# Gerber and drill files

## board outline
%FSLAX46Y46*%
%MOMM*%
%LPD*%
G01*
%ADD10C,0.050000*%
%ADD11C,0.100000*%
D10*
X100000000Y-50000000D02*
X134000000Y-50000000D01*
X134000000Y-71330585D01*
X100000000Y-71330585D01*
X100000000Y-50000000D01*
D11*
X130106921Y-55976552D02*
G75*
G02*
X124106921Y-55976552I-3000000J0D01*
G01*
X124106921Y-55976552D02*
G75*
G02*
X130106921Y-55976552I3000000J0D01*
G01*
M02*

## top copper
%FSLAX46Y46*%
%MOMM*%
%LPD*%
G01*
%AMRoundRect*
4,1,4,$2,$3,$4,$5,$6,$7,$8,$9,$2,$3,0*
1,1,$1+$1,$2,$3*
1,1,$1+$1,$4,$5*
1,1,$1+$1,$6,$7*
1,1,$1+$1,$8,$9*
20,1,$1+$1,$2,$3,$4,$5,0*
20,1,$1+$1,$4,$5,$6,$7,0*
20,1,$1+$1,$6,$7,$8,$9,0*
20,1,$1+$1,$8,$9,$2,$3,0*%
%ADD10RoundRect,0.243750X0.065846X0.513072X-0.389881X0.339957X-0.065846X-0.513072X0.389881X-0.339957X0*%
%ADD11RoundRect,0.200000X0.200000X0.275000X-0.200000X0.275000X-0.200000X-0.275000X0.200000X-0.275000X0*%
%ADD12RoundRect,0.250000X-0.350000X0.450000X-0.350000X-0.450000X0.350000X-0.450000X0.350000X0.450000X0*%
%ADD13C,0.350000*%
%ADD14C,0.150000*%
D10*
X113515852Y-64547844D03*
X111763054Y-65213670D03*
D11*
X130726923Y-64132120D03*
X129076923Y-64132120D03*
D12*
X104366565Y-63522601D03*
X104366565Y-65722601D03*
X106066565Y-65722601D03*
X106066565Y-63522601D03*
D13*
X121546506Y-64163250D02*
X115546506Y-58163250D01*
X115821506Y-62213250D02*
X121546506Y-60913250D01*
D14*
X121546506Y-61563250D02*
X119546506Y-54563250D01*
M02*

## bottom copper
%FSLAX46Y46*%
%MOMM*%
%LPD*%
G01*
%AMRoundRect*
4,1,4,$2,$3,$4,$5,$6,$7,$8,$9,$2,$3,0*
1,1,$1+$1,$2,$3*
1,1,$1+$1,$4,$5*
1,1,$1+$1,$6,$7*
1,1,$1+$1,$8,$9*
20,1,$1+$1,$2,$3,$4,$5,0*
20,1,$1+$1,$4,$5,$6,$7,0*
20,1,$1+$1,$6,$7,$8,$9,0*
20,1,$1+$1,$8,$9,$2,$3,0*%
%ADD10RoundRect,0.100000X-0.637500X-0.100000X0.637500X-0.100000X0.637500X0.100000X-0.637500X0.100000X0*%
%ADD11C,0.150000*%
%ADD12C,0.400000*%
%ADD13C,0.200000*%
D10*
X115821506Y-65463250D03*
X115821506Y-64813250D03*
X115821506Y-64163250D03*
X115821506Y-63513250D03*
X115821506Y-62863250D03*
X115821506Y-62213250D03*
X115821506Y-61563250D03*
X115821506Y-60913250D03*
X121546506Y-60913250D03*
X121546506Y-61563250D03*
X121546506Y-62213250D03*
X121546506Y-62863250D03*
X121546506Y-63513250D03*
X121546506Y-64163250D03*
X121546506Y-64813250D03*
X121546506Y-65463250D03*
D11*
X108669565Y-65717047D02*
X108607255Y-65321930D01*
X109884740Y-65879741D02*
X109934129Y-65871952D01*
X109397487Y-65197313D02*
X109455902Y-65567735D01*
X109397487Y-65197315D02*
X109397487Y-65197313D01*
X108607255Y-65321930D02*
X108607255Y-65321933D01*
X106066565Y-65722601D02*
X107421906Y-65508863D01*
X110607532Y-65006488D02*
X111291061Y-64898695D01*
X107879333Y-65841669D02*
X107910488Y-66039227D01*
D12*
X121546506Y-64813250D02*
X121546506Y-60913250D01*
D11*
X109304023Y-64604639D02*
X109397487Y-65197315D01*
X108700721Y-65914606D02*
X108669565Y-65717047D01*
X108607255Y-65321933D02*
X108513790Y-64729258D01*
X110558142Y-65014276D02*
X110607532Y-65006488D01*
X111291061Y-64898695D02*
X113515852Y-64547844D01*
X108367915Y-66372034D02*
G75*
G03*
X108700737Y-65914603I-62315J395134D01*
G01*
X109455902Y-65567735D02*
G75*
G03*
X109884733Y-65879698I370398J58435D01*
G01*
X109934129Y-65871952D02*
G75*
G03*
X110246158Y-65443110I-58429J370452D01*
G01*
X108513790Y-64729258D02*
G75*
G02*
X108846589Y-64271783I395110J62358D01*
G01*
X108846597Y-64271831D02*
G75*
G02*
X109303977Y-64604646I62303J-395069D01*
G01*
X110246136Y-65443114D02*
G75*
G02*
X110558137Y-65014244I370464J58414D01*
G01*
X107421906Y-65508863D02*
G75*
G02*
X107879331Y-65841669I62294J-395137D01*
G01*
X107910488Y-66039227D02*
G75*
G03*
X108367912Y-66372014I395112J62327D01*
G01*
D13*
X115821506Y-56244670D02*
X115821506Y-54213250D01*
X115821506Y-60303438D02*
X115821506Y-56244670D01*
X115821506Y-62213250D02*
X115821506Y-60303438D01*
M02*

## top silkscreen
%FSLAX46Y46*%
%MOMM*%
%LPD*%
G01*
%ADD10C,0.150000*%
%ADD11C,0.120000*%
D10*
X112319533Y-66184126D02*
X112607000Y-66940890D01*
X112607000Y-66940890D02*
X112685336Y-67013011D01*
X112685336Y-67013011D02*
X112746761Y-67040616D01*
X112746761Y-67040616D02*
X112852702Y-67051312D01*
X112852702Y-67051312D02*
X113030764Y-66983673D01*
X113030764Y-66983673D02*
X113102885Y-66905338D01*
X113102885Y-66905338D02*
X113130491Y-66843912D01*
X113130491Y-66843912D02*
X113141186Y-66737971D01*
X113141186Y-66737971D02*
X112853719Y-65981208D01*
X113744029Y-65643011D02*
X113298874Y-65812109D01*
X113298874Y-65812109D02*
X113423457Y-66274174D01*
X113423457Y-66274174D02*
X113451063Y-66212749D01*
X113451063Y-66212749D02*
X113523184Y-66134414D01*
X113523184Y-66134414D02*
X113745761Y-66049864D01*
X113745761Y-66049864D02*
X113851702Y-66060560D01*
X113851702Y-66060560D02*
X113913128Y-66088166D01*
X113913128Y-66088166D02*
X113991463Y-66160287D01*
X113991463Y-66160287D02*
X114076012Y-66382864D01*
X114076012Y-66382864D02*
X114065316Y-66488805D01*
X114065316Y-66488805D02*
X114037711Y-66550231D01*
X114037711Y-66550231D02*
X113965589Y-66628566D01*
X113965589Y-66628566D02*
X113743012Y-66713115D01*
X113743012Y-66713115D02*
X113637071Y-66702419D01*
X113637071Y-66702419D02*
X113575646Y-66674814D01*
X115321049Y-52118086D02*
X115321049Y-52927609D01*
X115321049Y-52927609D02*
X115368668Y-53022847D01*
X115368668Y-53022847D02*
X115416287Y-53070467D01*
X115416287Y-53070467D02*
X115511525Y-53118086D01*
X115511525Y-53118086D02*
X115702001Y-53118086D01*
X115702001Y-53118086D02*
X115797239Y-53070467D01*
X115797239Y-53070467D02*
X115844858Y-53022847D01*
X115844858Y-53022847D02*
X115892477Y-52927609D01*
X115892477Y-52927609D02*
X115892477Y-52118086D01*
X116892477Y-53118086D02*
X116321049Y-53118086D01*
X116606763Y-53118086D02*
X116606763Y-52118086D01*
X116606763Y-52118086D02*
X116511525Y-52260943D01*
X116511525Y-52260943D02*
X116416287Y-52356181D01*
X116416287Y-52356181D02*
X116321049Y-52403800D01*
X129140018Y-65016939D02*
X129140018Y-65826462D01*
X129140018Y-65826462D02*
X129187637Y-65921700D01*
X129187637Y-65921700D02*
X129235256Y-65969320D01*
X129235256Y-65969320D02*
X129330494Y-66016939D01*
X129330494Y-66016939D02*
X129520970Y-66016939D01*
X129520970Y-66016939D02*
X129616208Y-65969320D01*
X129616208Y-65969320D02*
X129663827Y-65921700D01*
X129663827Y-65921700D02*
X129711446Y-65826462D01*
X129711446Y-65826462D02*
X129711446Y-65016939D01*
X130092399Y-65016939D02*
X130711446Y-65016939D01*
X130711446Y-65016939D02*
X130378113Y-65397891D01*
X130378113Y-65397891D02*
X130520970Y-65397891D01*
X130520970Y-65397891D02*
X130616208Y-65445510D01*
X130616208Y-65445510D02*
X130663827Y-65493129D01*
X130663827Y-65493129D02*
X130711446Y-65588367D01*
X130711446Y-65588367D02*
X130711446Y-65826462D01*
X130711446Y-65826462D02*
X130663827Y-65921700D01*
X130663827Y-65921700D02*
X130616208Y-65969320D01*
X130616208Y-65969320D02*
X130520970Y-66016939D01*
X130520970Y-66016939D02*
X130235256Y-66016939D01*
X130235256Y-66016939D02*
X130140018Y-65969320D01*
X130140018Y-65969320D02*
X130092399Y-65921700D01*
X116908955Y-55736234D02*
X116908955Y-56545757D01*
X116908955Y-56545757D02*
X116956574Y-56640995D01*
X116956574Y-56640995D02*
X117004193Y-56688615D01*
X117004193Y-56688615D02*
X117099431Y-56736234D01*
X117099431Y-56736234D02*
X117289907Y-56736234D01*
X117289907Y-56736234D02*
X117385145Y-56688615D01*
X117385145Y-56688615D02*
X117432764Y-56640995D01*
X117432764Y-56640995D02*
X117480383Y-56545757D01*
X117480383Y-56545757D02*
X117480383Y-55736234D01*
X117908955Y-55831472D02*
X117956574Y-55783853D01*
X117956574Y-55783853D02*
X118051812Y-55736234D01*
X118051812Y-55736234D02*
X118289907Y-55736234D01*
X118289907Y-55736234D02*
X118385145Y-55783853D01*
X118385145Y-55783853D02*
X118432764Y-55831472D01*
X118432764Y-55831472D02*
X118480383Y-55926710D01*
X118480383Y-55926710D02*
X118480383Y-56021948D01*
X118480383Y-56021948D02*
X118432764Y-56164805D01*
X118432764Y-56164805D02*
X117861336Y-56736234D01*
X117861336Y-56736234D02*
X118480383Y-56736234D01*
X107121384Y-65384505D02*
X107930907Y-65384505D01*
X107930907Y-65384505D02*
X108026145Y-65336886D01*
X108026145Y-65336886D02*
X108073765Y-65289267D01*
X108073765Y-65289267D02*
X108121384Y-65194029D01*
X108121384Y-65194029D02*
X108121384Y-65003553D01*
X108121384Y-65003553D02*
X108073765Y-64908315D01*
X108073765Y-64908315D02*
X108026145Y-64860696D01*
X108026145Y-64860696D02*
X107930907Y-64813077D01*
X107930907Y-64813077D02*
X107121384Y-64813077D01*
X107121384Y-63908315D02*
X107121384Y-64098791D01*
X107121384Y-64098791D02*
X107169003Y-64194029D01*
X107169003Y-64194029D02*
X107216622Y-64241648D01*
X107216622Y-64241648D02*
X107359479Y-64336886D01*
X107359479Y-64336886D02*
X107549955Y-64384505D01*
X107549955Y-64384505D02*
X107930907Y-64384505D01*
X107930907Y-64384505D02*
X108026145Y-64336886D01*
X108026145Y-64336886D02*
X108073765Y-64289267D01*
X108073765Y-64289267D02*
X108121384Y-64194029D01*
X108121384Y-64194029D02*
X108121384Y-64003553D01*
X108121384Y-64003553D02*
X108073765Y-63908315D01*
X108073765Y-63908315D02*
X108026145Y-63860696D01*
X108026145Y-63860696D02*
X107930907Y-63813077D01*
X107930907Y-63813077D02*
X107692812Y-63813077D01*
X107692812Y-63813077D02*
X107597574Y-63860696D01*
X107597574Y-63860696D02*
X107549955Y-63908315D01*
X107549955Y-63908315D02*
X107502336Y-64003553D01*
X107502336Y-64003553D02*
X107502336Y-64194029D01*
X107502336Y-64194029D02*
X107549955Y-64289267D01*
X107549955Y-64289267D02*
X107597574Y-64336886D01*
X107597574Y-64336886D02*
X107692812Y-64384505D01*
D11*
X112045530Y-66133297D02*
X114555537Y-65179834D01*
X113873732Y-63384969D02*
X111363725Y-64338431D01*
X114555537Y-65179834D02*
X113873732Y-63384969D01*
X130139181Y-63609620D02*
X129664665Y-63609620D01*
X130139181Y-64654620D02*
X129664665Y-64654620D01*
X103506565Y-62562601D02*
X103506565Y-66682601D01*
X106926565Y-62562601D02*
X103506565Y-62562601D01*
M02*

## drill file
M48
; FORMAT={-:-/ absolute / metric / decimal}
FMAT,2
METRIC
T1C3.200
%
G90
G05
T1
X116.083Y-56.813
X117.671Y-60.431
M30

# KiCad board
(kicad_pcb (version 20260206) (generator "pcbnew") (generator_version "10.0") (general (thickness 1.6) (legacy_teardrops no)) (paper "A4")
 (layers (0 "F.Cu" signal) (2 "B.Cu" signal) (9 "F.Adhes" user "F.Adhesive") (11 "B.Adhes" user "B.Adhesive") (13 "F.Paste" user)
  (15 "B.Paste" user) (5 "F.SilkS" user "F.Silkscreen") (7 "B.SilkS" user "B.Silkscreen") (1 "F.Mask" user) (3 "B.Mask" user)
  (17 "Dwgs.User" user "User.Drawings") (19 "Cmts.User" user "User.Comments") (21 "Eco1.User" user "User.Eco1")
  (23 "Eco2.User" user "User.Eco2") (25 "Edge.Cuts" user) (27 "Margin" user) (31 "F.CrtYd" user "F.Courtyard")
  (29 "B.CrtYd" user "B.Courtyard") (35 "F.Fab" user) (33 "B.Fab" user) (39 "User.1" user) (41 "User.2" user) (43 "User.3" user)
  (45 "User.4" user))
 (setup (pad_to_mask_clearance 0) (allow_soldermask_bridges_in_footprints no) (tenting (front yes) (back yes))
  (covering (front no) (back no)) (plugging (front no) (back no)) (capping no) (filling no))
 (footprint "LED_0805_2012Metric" (layer "F.Cu") (at 112.639453 64.880757 -159.2)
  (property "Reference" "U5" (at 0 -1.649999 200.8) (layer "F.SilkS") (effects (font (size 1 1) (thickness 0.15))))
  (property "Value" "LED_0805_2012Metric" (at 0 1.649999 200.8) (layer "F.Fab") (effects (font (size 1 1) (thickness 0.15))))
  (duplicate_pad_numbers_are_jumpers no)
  (fp_line (start 1 -0.96) (end -1.685 -0.96) (stroke (width 0.12) (type solid)) (layer "F.SilkS"))
  (fp_line (start -1.685 0.96) (end 1 0.96) (stroke (width 0.12) (type solid)) (layer "F.SilkS"))
  (fp_line (start -1.685 -0.96) (end -1.685 0.96) (stroke (width 0.12) (type solid)) (layer "F.SilkS"))
  (pad "1" smd roundrect (at -0.9375 0 200.8) (size 0.975 1.4) (layers "F.Cu" "F.Mask" "F.Paste") (roundrect_rratio 0.25) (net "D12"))
  (pad "2" smd roundrect (at 0.9375 0 200.8) (size 0.975 1.4) (layers "F.Cu" "F.Mask" "F.Paste") (roundrect_rratio 0.25) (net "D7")))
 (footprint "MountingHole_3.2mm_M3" (layer "F.Cu") (at 116.082954 56.813267)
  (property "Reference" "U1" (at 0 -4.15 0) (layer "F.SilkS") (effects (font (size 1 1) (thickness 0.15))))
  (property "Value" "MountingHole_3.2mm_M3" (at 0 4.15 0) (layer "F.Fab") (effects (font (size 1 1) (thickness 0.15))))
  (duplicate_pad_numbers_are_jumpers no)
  (pad "" np_thru_hole circle (at 0 0) (size 3.2 3.2) (drill 3.2) (layers "*.Cu" "*.Mask")))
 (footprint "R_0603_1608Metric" (layer "F.Cu") (at 129.901923 64.13212 180)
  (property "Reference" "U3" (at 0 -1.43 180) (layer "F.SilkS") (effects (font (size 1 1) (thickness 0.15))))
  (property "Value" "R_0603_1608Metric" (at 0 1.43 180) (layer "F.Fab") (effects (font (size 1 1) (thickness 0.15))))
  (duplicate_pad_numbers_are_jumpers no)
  (fp_line (start -0.237258 0.5225) (end 0.237258 0.5225) (stroke (width 0.12) (type solid)) (layer "F.SilkS"))
  (fp_line (start -0.237258 -0.5225) (end 0.237258 -0.5225) (stroke (width 0.12) (type solid)) (layer "F.SilkS"))
  (pad "1" smd roundrect (at -0.825 0 180) (size 0.8 0.95) (layers "F.Cu" "F.Mask" "F.Paste") (roundrect_rratio 0.25) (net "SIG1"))
  (pad "2" smd roundrect (at 0.825 0 180) (size 0.8 0.95) (layers "F.Cu" "F.Mask" "F.Paste") (roundrect_rratio 0.25)))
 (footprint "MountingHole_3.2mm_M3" (layer "F.Cu") (at 117.67086 60.431415)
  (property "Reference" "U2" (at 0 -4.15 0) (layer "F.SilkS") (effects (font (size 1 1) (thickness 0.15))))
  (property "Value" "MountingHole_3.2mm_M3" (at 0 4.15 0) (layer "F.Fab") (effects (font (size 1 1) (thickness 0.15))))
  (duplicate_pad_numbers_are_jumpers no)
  (pad "" np_thru_hole circle (at 0 0) (size 3.2 3.2) (drill 3.2) (layers "*.Cu" "*.Mask")))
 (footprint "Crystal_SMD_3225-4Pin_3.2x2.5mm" (layer "F.Cu") (at 105.216565 64.622601 -90)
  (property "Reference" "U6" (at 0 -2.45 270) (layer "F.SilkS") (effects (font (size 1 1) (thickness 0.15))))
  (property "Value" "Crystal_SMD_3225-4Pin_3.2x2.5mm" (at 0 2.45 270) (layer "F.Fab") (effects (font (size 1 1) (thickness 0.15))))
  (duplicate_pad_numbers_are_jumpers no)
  (fp_line (start -2.06 1.71) (end 2.06 1.71) (stroke (width 0.12) (type solid)) (layer "F.SilkS"))
  (fp_line (start -2.06 -1.71) (end -2.06 1.71) (stroke (width 0.12) (type solid)) (layer "F.SilkS"))
  (pad "1" smd roundrect (at -1.1 0.85 270) (size 1.4 1.2) (layers "F.Cu" "F.Mask" "F.Paste") (roundrect_rratio 0.208333) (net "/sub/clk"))
  (pad "2" smd roundrect (at 1.1 0.85 270) (size 1.4 1.2) (layers "F.Cu" "F.Mask" "F.Paste") (roundrect_rratio 0.208333) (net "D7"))
  (pad "3" smd roundrect (at 1.1 -0.85 270) (size 1.4 1.2) (layers "F.Cu" "F.Mask" "F.Paste") (roundrect_rratio 0.208333) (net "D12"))
  (pad "4" smd roundrect (at -1.1 -0.85 270) (size 1.4 1.2) (layers "F.Cu" "F.Mask" "F.Paste") (roundrect_rratio 0.208333) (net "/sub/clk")))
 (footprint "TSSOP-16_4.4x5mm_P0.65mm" (layer "B.Cu") (at 118.684006 63.18825)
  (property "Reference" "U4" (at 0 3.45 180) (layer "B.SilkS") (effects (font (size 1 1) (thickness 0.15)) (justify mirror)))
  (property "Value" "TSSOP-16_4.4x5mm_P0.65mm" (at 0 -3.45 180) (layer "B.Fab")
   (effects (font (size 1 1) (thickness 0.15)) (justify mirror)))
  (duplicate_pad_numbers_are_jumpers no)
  (pad "1" smd roundrect (at -2.8625 2.275) (size 1.475 0.4) (layers "B.Cu" "B.Mask" "B.Paste") (roundrect_rratio 0.25) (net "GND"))
  (pad "2" smd roundrect (at -2.8625 1.625) (size 1.475 0.4) (layers "B.Cu" "B.Mask" "B.Paste") (roundrect_rratio 0.25) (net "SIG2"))
  (pad "3" smd roundrect (at -2.8625 0.975) (size 1.475 0.4) (layers "B.Cu" "B.Mask" "B.Paste") (roundrect_rratio 0.25) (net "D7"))
  (pad "4" smd roundrect (at -2.8625 0.325) (size 1.475 0.4) (layers "B.Cu" "B.Mask" "B.Paste") (roundrect_rratio 0.25) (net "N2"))
  (pad "5" smd roundrect (at -2.8625 -0.325) (size 1.475 0.4) (layers "B.Cu" "B.Mask" "B.Paste") (roundrect_rratio 0.25) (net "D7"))
  (pad "6" smd roundrect (at -2.8625 -0.975) (size 1.475 0.4) (layers "B.Cu" "B.Mask" "B.Paste") (roundrect_rratio 0.25) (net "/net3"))
  (pad "7" smd roundrect (at -2.8625 -1.625) (size 1.475 0.4) (layers "B.Cu" "B.Mask" "B.Paste") (roundrect_rratio 0.25))
  (pad "8" smd roundrect (at -2.8625 -2.275) (size 1.475 0.4) (layers "B.Cu" "B.Mask" "B.Paste") (roundrect_rratio 0.25) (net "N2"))
  (pad "9" smd roundrect (at 2.8625 -2.275) (size 1.475 0.4) (layers "B.Cu" "B.Mask" "B.Paste") (roundrect_rratio 0.25))
  (pad "10" smd roundrect (at 2.8625 -1.625) (size 1.475 0.4) (layers "B.Cu" "B.Mask" "B.Paste") (roundrect_rratio 0.25) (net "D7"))
  (pad "11" smd roundrect (at 2.8625 -0.975) (size 1.475 0.4) (layers "B.Cu" "B.Mask" "B.Paste") (roundrect_rratio 0.25) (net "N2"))
  (pad "12" smd roundrect (at 2.8625 -0.325) (size 1.475 0.4) (layers "B.Cu" "B.Mask" "B.Paste") (roundrect_rratio 0.25))
  (pad "13" smd roundrect (at 2.8625 0.325) (size 1.475 0.4) (layers "B.Cu" "B.Mask" "B.Paste") (roundrect_rratio 0.25))
  (pad "14" smd roundrect (at 2.8625 0.975) (size 1.475 0.4) (layers "B.Cu" "B.Mask" "B.Paste") (roundrect_rratio 0.25) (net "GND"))
  (pad "15" smd roundrect (at 2.8625 1.625) (size 1.475 0.4) (layers "B.Cu" "B.Mask" "B.Paste") (roundrect_rratio 0.25) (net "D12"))
  (pad "16" smd roundrect (at 2.8625 2.275) (size 1.475 0.4) (layers "B.Cu" "B.Mask" "B.Paste") (roundrect_rratio 0.25)))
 (gr_rect (start 100 50) (end 134 71.330585) (stroke (width 0.05) (type default)) (fill no) (layer "Edge.Cuts"))
 (gr_circle (center 127.106921 55.976552) (end 130.106921 55.976552) (stroke (width 0.1) (type default)) (fill no) (layer "Edge.Cuts"))
 (segment (start 108.669565 65.717047) (end 108.607255 65.32193) (width 0.15) (layer "B.Cu") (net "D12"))
 (segment (start 109.88474 65.879741) (end 109.934129 65.871952) (width 0.15) (layer "B.Cu") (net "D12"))
 (segment (start 109.397487 65.197313) (end 109.455902 65.567735) (width 0.15) (layer "B.Cu") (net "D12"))
 (segment (start 109.397487 65.197315) (end 109.397487 65.197313) (width 0.15) (layer "B.Cu") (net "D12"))
 (segment (start 108.607255 65.32193) (end 108.607255 65.321933) (width 0.15) (layer "B.Cu") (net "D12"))
 (segment (start 106.066565 65.722601) (end 107.421906 65.508863) (width 0.15) (layer "B.Cu") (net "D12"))
 (segment (start 110.607532 65.006488) (end 111.291061 64.898695) (width 0.15) (layer "B.Cu") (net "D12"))
 (segment (start 107.879333 65.841669) (end 107.910488 66.039227) (width 0.15) (layer "B.Cu") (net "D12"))
 (segment (start 121.546506 64.81325) (end 121.546506 60.91325) (width 0.4) (layer "B.Cu") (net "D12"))
 (segment (start 109.304023 64.604639) (end 109.397487 65.197315) (width 0.15) (layer "B.Cu") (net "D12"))
 (segment (start 108.700721 65.914606) (end 108.669565 65.717047) (width 0.15) (layer "B.Cu") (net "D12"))
 (segment (start 108.607255 65.321933) (end 108.51379 64.729258) (width 0.15) (layer "B.Cu") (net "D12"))
 (segment (start 110.558142 65.014276) (end 110.607532 65.006488) (width 0.15) (layer "B.Cu") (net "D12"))
 (segment (start 111.291061 64.898695) (end 113.515852 64.547844) (width 0.15) (layer "B.Cu") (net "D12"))
 (arc (start 108.367915 66.372034) (mid 108.629054 66.212246) (end 108.700721 65.914606) (width 0.15) (layer "B.Cu") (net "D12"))
 (arc (start 109.455902 65.567735) (mid 109.605702 65.812553) (end 109.88474 65.879741) (width 0.15) (layer "B.Cu") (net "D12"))
 (arc (start 109.934129 65.871952) (mid 110.178948 65.722151) (end 110.246136 65.443114) (width 0.15) (layer "B.Cu") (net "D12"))
 (arc (start 108.51379 64.729258) (mid 108.585457 64.431618) (end 108.846597 64.271831) (width 0.15) (layer "B.Cu") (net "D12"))
 (arc (start 108.846597 64.271831) (mid 109.144236 64.343499) (end 109.304023 64.604639) (width 0.15) (layer "B.Cu") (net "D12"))
 (arc (start 110.246136 65.443114) (mid 110.313324 65.164076) (end 110.558142 65.014276) (width 0.15) (layer "B.Cu") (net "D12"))
 (arc (start 107.421906 65.508863) (mid 107.719545 65.58053) (end 107.879333 65.841669) (width 0.15) (layer "B.Cu") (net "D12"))
 (arc (start 107.910488 66.039227) (mid 108.070275 66.300367) (end 108.367915 66.372034) (width 0.15) (layer "B.Cu") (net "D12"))
 (segment (start 121.546506 64.16325) (end 115.546506 58.16325) (width 0.35) (layer "F.Cu") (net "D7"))
 (segment (start 115.821506 62.21325) (end 121.546506 60.91325) (width 0.35) (layer "F.Cu") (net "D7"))
 (segment (start 121.546506 61.56325) (end 119.546506 54.56325) (width 0.15) (layer "F.Cu") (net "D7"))
 (segment (start 115.821506 56.24467) (end 115.821506 54.21325) (width 0.2) (layer "B.Cu") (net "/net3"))
 (segment (start 115.821506 60.303438) (end 115.821506 56.24467) (width 0.2) (layer "B.Cu") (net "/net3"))
 (segment (start 115.821506 62.21325) (end 115.821506 60.303438) (width 0.2) (layer "B.Cu") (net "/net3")))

